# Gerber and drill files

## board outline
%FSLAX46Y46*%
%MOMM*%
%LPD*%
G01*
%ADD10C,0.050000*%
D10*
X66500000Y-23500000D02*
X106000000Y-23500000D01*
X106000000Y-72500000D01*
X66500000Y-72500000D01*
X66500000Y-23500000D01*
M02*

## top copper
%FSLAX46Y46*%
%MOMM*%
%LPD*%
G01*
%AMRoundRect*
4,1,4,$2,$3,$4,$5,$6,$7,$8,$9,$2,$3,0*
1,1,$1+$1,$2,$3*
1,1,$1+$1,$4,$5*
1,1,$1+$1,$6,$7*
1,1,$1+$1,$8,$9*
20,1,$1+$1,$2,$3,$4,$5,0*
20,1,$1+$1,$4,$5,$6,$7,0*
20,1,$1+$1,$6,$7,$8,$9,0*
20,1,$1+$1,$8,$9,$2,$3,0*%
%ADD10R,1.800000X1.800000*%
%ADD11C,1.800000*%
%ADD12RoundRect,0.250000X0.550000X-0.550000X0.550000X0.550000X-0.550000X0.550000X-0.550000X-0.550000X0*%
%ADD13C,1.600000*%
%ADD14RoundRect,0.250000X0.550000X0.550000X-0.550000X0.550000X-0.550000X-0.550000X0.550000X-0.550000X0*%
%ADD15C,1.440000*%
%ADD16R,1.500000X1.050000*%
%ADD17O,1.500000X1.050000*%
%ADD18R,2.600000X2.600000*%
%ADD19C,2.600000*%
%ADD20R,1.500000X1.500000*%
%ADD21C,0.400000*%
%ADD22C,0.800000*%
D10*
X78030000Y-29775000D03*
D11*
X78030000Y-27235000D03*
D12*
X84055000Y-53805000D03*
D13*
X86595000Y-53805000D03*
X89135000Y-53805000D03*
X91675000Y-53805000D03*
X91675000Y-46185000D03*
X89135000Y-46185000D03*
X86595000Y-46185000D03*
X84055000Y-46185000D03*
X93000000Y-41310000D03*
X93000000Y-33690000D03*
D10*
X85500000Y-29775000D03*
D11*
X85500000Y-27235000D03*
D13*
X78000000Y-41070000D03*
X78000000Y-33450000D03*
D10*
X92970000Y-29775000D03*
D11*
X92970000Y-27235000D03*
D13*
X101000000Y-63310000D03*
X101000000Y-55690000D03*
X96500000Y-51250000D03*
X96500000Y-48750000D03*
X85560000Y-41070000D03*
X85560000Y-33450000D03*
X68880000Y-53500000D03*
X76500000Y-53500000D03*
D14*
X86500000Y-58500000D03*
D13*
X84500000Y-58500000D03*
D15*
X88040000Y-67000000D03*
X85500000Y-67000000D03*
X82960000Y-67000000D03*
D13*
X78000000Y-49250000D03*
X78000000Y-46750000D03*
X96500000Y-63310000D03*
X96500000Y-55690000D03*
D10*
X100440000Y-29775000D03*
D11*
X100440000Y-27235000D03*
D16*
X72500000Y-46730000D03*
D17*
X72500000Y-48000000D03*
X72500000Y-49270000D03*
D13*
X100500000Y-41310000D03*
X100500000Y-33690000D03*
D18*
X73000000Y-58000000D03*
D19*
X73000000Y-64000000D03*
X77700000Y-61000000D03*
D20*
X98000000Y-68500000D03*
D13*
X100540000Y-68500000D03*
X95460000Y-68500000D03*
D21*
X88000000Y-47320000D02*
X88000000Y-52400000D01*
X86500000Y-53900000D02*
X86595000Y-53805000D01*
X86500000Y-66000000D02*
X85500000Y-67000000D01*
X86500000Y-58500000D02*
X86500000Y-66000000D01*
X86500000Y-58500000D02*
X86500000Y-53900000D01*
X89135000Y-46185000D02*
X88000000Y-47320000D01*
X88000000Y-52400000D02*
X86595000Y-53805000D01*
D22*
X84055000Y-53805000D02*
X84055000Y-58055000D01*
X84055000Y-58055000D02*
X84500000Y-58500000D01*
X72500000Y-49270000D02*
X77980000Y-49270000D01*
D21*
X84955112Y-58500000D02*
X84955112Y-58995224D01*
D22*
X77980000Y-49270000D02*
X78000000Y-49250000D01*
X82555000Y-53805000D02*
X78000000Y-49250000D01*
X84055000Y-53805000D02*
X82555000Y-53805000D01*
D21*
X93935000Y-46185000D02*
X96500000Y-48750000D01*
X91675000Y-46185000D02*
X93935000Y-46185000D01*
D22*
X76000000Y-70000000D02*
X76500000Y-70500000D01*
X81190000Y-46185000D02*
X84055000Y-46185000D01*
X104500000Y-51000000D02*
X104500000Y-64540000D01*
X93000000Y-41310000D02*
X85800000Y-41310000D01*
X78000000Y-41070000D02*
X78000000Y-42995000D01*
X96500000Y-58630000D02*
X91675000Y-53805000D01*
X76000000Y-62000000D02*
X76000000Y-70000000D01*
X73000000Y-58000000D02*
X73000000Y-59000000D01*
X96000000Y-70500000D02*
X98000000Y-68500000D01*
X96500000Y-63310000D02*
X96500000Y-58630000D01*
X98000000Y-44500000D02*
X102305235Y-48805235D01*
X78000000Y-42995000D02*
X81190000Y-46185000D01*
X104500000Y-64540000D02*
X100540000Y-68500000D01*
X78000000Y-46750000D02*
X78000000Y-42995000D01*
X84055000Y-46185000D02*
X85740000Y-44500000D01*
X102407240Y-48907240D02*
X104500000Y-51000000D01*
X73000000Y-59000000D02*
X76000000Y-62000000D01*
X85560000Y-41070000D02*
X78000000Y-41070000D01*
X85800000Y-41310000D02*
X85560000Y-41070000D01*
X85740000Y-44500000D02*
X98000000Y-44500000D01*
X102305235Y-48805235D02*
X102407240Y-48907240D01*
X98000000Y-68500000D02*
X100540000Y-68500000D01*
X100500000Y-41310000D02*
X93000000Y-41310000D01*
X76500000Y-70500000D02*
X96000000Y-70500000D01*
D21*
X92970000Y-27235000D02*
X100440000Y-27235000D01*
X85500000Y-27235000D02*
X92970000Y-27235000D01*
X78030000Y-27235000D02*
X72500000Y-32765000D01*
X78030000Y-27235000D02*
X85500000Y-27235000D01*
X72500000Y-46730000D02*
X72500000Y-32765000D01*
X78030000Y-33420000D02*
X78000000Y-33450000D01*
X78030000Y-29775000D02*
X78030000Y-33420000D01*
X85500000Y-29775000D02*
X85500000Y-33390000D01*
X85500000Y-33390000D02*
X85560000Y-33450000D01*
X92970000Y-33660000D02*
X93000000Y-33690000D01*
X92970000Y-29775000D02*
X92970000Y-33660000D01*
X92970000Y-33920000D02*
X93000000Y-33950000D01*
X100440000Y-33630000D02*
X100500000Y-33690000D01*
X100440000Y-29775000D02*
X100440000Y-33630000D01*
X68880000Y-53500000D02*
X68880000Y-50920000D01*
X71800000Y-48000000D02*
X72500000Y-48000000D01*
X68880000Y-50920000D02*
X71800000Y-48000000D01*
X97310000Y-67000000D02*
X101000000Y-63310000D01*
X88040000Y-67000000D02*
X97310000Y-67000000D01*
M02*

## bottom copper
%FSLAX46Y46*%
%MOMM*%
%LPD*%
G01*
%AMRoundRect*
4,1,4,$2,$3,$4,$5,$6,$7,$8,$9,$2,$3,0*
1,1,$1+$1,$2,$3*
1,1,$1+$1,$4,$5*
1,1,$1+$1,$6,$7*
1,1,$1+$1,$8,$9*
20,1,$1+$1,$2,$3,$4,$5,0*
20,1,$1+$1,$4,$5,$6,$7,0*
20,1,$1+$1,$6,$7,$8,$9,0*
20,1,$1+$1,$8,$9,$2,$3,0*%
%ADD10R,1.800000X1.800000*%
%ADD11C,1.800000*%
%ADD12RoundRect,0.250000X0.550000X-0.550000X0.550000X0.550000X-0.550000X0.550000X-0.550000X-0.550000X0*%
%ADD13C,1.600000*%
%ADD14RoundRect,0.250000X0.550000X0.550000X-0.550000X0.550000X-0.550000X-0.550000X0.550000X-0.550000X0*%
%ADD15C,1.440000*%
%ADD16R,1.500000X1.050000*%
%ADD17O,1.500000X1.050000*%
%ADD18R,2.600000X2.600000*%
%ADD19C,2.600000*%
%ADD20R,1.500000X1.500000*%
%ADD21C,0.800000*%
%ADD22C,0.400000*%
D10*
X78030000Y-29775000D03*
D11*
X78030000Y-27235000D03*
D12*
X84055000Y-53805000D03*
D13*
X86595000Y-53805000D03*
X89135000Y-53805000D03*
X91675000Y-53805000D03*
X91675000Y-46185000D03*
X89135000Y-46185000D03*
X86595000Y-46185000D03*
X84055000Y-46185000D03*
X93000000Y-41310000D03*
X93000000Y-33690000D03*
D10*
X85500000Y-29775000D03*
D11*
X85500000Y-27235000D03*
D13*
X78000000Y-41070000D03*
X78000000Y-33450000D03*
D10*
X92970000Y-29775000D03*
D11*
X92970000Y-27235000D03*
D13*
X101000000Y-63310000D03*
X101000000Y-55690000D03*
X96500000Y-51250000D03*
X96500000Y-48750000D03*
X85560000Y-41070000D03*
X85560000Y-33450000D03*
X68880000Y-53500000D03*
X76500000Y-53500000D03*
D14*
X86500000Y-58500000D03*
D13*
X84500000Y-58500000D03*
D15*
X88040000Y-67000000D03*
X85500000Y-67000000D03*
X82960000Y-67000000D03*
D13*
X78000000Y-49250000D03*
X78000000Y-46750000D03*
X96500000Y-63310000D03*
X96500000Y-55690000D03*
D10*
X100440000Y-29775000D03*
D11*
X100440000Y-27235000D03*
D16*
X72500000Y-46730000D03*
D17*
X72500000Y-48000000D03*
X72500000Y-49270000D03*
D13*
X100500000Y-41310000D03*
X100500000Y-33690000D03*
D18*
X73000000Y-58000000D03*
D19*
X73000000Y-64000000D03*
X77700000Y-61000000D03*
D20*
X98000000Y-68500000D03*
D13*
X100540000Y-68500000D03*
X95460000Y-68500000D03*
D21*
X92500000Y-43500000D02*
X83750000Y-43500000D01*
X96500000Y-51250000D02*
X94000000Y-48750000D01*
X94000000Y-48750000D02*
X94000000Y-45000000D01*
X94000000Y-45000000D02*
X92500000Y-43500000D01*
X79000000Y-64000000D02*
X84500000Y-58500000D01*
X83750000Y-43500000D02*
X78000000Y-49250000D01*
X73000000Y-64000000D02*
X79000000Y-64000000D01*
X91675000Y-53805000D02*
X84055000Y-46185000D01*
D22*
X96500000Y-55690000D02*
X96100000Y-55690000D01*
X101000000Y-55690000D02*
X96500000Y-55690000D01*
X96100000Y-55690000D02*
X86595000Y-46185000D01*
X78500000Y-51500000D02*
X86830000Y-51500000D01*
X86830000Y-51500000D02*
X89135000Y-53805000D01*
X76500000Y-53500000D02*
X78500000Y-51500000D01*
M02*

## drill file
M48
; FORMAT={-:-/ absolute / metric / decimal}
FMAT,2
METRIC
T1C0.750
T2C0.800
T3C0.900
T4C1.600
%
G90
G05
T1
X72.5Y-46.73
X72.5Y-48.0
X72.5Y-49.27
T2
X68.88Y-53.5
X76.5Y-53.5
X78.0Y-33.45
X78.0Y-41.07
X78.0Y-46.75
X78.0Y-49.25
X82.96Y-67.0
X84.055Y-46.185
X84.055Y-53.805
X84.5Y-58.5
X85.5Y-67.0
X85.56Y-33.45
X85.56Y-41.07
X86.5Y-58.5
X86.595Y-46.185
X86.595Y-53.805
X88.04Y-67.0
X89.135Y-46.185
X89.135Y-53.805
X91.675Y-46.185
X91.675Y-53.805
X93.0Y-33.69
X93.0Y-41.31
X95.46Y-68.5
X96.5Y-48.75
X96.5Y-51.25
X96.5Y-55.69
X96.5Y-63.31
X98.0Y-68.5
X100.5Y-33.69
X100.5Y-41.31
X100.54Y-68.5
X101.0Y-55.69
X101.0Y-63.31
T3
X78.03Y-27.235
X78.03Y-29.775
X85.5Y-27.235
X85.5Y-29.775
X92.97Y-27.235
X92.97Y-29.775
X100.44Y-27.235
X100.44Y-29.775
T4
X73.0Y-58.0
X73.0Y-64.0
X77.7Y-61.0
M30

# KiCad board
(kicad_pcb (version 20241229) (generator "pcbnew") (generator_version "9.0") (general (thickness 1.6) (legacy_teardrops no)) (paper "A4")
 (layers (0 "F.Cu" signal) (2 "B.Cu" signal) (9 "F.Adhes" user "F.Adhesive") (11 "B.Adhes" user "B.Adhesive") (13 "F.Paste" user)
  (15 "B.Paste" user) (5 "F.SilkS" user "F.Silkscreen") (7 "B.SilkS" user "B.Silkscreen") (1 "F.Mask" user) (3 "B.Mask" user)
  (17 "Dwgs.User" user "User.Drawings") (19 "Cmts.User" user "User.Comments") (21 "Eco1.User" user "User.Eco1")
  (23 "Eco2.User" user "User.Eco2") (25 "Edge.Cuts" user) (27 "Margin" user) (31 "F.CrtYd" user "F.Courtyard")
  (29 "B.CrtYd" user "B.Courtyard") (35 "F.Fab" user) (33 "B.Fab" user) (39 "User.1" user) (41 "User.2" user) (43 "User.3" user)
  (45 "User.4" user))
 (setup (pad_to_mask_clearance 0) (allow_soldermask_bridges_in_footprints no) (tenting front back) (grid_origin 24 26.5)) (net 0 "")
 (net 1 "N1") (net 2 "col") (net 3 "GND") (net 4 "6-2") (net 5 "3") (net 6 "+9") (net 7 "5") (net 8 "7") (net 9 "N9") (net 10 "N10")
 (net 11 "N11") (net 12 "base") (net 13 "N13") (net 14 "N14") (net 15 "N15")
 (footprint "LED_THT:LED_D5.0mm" (layer "F.Cu") (at 78.03 29.775 90)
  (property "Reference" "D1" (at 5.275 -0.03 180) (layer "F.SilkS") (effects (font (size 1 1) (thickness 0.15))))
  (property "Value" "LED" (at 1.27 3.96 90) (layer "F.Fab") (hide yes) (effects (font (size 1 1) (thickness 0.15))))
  (pad "1" thru_hole rect (at 0 0 90) (size 1.8 1.8) (drill 0.9) (layers "*.Cu" "*.Mask") (remove_unused_layers no) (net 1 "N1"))
  (pad "2" thru_hole circle (at 2.54 0 90) (size 1.8 1.8) (drill 0.9) (layers "*.Cu" "*.Mask") (remove_unused_layers no) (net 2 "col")))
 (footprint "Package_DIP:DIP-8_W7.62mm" (layer "F.Cu") (at 84.055 53.805 90)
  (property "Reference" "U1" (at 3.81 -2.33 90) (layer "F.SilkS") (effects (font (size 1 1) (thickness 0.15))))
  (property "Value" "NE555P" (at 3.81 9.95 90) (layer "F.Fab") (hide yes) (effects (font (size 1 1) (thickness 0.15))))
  (pad "1" thru_hole roundrect (at 0 0 90) (size 1.6 1.6) (drill 0.8) (layers "*.Cu" "*.Mask") (remove_unused_layers no)
   (roundrect_rratio 0.15625) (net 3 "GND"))
  (pad "2" thru_hole circle (at 0 2.54 90) (size 1.6 1.6) (drill 0.8) (layers "*.Cu" "*.Mask") (remove_unused_layers no) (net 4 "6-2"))
  (pad "3" thru_hole circle (at 0 5.08 90) (size 1.6 1.6) (drill 0.8) (layers "*.Cu" "*.Mask") (remove_unused_layers no) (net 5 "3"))
  (pad "4" thru_hole circle (at 0 7.62 90) (size 1.6 1.6) (drill 0.8) (layers "*.Cu" "*.Mask") (remove_unused_layers no) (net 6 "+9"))
  (pad "5" thru_hole circle (at 7.62 7.62 90) (size 1.6 1.6) (drill 0.8) (layers "*.Cu" "*.Mask") (remove_unused_layers no) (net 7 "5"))
  (pad "6" thru_hole circle (at 7.62 5.08 90) (size 1.6 1.6) (drill 0.8) (layers "*.Cu" "*.Mask") (remove_unused_layers no) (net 4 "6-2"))
  (pad "7" thru_hole circle (at 7.62 2.54 90) (size 1.6 1.6) (drill 0.8) (layers "*.Cu" "*.Mask") (remove_unused_layers no) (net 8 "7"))
  (pad "8" thru_hole circle (at 7.62 0 90) (size 1.6 1.6) (drill 0.8) (layers "*.Cu" "*.Mask") (remove_unused_layers no) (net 6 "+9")))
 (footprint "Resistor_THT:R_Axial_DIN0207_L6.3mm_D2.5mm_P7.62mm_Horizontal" (layer "F.Cu") (at 93 41.31 90)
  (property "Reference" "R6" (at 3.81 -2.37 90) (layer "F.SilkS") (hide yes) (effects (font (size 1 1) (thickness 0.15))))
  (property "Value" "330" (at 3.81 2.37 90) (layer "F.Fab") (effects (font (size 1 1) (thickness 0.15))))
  (pad "1" thru_hole circle (at 0 0 90) (size 1.6 1.6) (drill 0.8) (layers "*.Cu" "*.Mask") (remove_unused_layers no) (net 6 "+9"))
  (pad "2" thru_hole circle (at 7.62 0 90) (size 1.6 1.6) (drill 0.8) (layers "*.Cu" "*.Mask") (remove_unused_layers no) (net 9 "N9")))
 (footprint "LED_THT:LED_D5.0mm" (layer "F.Cu") (at 85.5 29.775 90)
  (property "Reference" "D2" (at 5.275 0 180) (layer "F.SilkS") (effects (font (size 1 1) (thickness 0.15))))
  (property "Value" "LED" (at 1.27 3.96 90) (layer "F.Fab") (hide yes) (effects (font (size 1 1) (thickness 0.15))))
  (pad "1" thru_hole rect (at 0 0 90) (size 1.8 1.8) (drill 0.9) (layers "*.Cu" "*.Mask") (remove_unused_layers no) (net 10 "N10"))
  (pad "2" thru_hole circle (at 2.54 0 90) (size 1.8 1.8) (drill 0.9) (layers "*.Cu" "*.Mask") (remove_unused_layers no) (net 2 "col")))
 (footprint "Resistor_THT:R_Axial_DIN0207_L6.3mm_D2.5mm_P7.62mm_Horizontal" (layer "F.Cu") (at 78 41.07 90)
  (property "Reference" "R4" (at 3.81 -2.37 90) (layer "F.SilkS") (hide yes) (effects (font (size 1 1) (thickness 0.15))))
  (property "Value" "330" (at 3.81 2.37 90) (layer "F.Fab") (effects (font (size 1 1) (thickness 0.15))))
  (pad "1" thru_hole circle (at 0 0 90) (size 1.6 1.6) (drill 0.8) (layers "*.Cu" "*.Mask") (remove_unused_layers no) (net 6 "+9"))
  (pad "2" thru_hole circle (at 7.62 0 90) (size 1.6 1.6) (drill 0.8) (layers "*.Cu" "*.Mask") (remove_unused_layers no) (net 1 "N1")))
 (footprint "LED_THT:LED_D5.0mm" (layer "F.Cu") (at 92.97 29.775 90)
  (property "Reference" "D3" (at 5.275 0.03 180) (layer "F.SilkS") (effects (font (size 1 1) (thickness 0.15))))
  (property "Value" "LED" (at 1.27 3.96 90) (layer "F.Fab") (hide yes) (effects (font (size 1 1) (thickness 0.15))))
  (pad "1" thru_hole rect (at 0 0 90) (size 1.8 1.8) (drill 0.9) (layers "*.Cu" "*.Mask") (remove_unused_layers no) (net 9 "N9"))
  (pad "2" thru_hole circle (at 2.54 0 90) (size 1.8 1.8) (drill 0.9) (layers "*.Cu" "*.Mask") (remove_unused_layers no) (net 2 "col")))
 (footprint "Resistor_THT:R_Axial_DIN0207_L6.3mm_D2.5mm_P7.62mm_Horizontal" (layer "F.Cu") (at 101 63.31 90)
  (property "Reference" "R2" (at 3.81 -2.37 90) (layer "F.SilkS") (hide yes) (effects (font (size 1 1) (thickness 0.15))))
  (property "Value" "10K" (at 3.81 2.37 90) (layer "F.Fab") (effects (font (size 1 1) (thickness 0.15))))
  (pad "1" thru_hole circle (at 0 0 90) (size 1.6 1.6) (drill 0.8) (layers "*.Cu" "*.Mask") (remove_unused_layers no) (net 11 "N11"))
  (pad "2" thru_hole circle (at 7.62 0 90) (size 1.6 1.6) (drill 0.8) (layers "*.Cu" "*.Mask") (remove_unused_layers no) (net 8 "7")))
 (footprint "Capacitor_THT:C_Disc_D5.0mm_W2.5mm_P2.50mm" (layer "F.Cu") (at 96.5 51.25 90)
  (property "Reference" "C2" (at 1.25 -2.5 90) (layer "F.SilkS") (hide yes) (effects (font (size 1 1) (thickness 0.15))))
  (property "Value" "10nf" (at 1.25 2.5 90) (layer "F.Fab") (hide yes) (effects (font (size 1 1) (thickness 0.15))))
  (pad "1" thru_hole circle (at 0 0 90) (size 1.6 1.6) (drill 0.8) (layers "*.Cu" "*.Mask") (remove_unused_layers no) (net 3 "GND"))
  (pad "2" thru_hole circle (at 2.5 0 90) (size 1.6 1.6) (drill 0.8) (layers "*.Cu" "*.Mask") (remove_unused_layers no) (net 7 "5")))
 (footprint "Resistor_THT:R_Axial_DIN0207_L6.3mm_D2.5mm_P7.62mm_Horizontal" (layer "F.Cu") (at 85.56 41.07 90)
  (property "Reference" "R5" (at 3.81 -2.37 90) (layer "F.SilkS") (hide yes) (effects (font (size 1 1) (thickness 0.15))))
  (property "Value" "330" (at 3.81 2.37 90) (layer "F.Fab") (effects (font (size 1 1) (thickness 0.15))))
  (pad "1" thru_hole circle (at 0 0 90) (size 1.6 1.6) (drill 0.8) (layers "*.Cu" "*.Mask") (remove_unused_layers no) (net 6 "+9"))
  (pad "2" thru_hole circle (at 7.62 0 90) (size 1.6 1.6) (drill 0.8) (layers "*.Cu" "*.Mask") (remove_unused_layers no) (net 10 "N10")))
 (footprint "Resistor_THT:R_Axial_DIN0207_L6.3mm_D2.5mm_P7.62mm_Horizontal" (layer "F.Cu") (at 68.88 53.5)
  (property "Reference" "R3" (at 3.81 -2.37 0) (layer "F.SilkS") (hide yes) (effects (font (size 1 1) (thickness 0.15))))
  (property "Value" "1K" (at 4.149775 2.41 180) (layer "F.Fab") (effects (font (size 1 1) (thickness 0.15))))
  (pad "1" thru_hole circle (at 0 0) (size 1.6 1.6) (drill 0.8) (layers "*.Cu" "*.Mask") (remove_unused_layers no) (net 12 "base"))
  (pad "2" thru_hole circle (at 7.62 0) (size 1.6 1.6) (drill 0.8) (layers "*.Cu" "*.Mask") (remove_unused_layers no) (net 5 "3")))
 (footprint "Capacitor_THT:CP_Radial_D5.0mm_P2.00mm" (layer "F.Cu") (at 86.5 58.5 180)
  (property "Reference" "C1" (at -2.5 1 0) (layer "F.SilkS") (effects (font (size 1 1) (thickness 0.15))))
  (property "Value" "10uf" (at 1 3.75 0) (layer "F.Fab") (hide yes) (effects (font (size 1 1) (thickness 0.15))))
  (pad "1" thru_hole roundrect (at 0 0 180) (size 1.6 1.6) (drill 0.8) (layers "*.Cu" "*.Mask") (remove_unused_layers no)
   (roundrect_rratio 0.15625) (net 4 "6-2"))
  (pad "2" thru_hole circle (at 2 0 180) (size 1.6 1.6) (drill 0.8) (layers "*.Cu" "*.Mask") (remove_unused_layers no) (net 3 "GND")))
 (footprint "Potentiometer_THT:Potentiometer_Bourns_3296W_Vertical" (layer "F.Cu") (at 88.04 67)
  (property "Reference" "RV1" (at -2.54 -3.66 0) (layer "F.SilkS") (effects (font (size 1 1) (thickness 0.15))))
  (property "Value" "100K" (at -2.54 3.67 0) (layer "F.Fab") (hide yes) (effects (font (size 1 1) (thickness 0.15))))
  (pad "1" thru_hole circle (at 0 0) (size 1.44 1.44) (drill 0.8) (layers "*.Cu" "*.Mask") (remove_unused_layers no) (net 11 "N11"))
  (pad "2" thru_hole circle (at -2.54 0) (size 1.44 1.44) (drill 0.8) (layers "*.Cu" "*.Mask") (remove_unused_layers no) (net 4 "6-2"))
  (pad "3" thru_hole circle (at -5.08 0) (size 1.44 1.44) (drill 0.8) (layers "*.Cu" "*.Mask") (remove_unused_layers no) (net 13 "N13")))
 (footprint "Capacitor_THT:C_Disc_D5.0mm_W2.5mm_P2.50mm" (layer "F.Cu") (at 78 49.25 90)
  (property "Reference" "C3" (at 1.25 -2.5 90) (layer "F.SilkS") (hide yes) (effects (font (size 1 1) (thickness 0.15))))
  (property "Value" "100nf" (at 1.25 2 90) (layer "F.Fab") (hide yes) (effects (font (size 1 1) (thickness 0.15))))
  (pad "1" thru_hole circle (at 0 0 90) (size 1.6 1.6) (drill 0.8) (layers "*.Cu" "*.Mask") (remove_unused_layers no) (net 3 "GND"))
  (pad "2" thru_hole circle (at 2.5 0 90) (size 1.6 1.6) (drill 0.8) (layers "*.Cu" "*.Mask") (remove_unused_layers no) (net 6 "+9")))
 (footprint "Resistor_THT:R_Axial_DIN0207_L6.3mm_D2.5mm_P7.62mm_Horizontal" (layer "F.Cu") (at 96.5 63.31 90)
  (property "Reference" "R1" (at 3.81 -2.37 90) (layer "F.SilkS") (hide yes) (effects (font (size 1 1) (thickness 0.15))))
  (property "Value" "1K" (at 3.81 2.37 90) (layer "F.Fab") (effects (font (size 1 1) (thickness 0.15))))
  (pad "1" thru_hole circle (at 0 0 90) (size 1.6 1.6) (drill 0.8) (layers "*.Cu" "*.Mask") (remove_unused_layers no) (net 6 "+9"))
  (pad "2" thru_hole circle (at 7.62 0 90) (size 1.6 1.6) (drill 0.8) (layers "*.Cu" "*.Mask") (remove_unused_layers no) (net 8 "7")))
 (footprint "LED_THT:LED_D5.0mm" (layer "F.Cu") (at 100.44 29.775 90)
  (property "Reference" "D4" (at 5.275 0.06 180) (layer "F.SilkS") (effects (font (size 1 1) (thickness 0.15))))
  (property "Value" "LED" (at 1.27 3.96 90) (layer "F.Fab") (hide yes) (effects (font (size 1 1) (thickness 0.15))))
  (pad "1" thru_hole rect (at 0 0 90) (size 1.8 1.8) (drill 0.9) (layers "*.Cu" "*.Mask") (remove_unused_layers no) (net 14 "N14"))
  (pad "2" thru_hole circle (at 2.54 0 90) (size 1.8 1.8) (drill 0.9) (layers "*.Cu" "*.Mask") (remove_unused_layers no) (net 2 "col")))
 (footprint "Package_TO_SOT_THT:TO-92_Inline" (layer "F.Cu") (at 72.5 46.73 -90)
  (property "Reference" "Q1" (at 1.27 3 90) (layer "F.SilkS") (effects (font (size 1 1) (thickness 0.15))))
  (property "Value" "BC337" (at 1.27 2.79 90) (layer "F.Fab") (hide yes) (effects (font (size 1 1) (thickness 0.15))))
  (pad "1" thru_hole rect (at 0 0 270) (size 1.05 1.5) (drill 0.75) (layers "*.Cu" "*.Mask") (remove_unused_layers no) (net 2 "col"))
  (pad "2" thru_hole oval (at 1.27 0 270) (size 1.05 1.5) (drill 0.75) (layers "*.Cu" "*.Mask") (remove_unused_layers no) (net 12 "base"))
  (pad "3" thru_hole oval (at 2.54 0 270) (size 1.05 1.5) (drill 0.75) (layers "*.Cu" "*.Mask") (remove_unused_layers no) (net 3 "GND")))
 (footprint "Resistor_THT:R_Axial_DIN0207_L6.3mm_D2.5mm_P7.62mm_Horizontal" (layer "F.Cu") (at 100.5 41.31 90)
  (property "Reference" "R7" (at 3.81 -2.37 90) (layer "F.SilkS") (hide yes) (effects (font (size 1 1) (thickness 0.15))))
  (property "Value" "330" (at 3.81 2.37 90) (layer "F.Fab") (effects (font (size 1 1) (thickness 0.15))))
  (pad "1" thru_hole circle (at 0 0 90) (size 1.6 1.6) (drill 0.8) (layers "*.Cu" "*.Mask") (remove_unused_layers no) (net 6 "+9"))
  (pad "2" thru_hole circle (at 7.62 0 90) (size 1.6 1.6) (drill 0.8) (layers "*.Cu" "*.Mask") (remove_unused_layers no) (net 14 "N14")))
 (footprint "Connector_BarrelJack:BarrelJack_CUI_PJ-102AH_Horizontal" (layer "F.Cu") (at 73 58)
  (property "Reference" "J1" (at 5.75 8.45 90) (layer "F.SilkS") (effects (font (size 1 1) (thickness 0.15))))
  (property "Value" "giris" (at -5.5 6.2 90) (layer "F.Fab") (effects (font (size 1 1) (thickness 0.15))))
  (pad "1" thru_hole rect (at 0 0) (size 2.6 2.6) (drill 1.6) (layers "*.Cu" "*.Mask") (remove_unused_layers no) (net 6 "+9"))
  (pad "2" thru_hole circle (at 0 6) (size 2.6 2.6) (drill 1.6) (layers "*.Cu" "*.Mask") (remove_unused_layers no) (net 3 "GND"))
  (pad "3" thru_hole circle (at 4.7 3) (size 2.6 2.6) (drill 1.6) (layers "*.Cu" "*.Mask") (remove_unused_layers no)))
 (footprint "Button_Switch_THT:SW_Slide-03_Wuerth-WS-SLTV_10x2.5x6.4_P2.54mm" (layer "F.Cu") (at 98 68.5 180)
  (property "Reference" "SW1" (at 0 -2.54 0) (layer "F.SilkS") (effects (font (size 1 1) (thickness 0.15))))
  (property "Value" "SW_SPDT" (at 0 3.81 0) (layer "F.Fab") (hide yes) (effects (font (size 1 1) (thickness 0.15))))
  (pad "1" thru_hole rect (at 0 0 180) (size 1.5 1.5) (drill 0.8) (layers "*.Cu" "*.Mask") (remove_unused_layers no) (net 6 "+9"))
  (pad "2" thru_hole circle (at -2.54 0 180) (size 1.6 1.6) (drill 0.8) (layers "*.Cu" "*.Mask") (remove_unused_layers no) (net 6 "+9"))
  (pad "3" thru_hole circle (at 2.54 0 180) (size 1.6 1.6) (drill 0.8) (layers "*.Cu" "*.Mask") (remove_unused_layers no) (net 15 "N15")))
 (gr_rect (start 66.5 23.5) (end 106 72.5) (stroke (width 0.05) (type default)) (fill no) (layer "Edge.Cuts"))
 (segment (start 88 47.32) (end 88 52.4) (width 0.4) (layer "F.Cu") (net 4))
 (segment (start 86.5 53.9) (end 86.595 53.805) (width 0.4) (layer "F.Cu") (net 4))
 (segment (start 86.5 66) (end 85.5 67) (width 0.4) (layer "F.Cu") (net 4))
 (segment (start 86.5 58.5) (end 86.5 66) (width 0.4) (layer "F.Cu") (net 4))
 (segment (start 86.5 58.5) (end 86.5 53.9) (width 0.4) (layer "F.Cu") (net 4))
 (segment (start 89.135 46.185) (end 88 47.32) (width 0.4) (layer "F.Cu") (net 4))
 (segment (start 88 52.4) (end 86.595 53.805) (width 0.4) (layer "F.Cu") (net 4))
 (segment (start 84.055 53.805) (end 84.055 58.055) (width 0.8) (layer "F.Cu") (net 3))
 (segment (start 84.055 58.055) (end 84.5 58.5) (width 0.8) (layer "F.Cu") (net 3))
 (segment (start 72.5 49.27) (end 77.98 49.27) (width 0.8) (layer "F.Cu") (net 3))
 (segment (start 84.955112 58.5) (end 84.955112 58.995224) (width 0.4) (layer "F.Cu") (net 3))
 (segment (start 77.98 49.27) (end 78 49.25) (width 0.8) (layer "F.Cu") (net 3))
 (segment (start 82.555 53.805) (end 78 49.25) (width 0.8) (layer "F.Cu") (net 3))
 (segment (start 84.055 53.805) (end 82.555 53.805) (width 0.8) (layer "F.Cu") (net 3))
 (segment (start 92.5 43.5) (end 83.75 43.5) (width 0.8) (layer "B.Cu") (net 3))
 (segment (start 96.5 51.25) (end 94 48.75) (width 0.8) (layer "B.Cu") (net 3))
 (segment (start 94 48.75) (end 94 45) (width 0.8) (layer "B.Cu") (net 3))
 (segment (start 94 45) (end 92.5 43.5) (width 0.8) (layer "B.Cu") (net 3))
 (segment (start 79 64) (end 84.5 58.5) (width 0.8) (layer "B.Cu") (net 3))
 (segment (start 83.75 43.5) (end 78 49.25) (width 0.8) (layer "B.Cu") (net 3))
 (segment (start 73 64) (end 79 64) (width 0.8) (layer "B.Cu") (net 3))
 (segment (start 93.935 46.185) (end 96.5 48.75) (width 0.4) (layer "F.Cu") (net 7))
 (segment (start 91.675 46.185) (end 93.935 46.185) (width 0.4) (layer "F.Cu") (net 7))
 (segment (start 76 70) (end 76.5 70.5) (width 0.8) (layer "F.Cu") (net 6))
 (segment (start 81.19 46.185) (end 84.055 46.185) (width 0.8) (layer "F.Cu") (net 6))
 (segment (start 104.5 51) (end 104.5 64.54) (width 0.8) (layer "F.Cu") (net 6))
 (segment (start 93 41.31) (end 85.8 41.31) (width 0.8) (layer "F.Cu") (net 6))
 (segment (start 78 41.07) (end 78 42.995) (width 0.8) (layer "F.Cu") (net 6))
 (segment (start 96.5 58.63) (end 91.675 53.805) (width 0.8) (layer "F.Cu") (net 6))
 (segment (start 76 62) (end 76 70) (width 0.8) (layer "F.Cu") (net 6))
 (segment (start 73 58) (end 73 59) (width 0.8) (layer "F.Cu") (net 6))
 (segment (start 96 70.5) (end 98 68.5) (width 0.8) (layer "F.Cu") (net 6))
 (segment (start 96.5 63.31) (end 96.5 58.63) (width 0.8) (layer "F.Cu") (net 6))
 (segment (start 98 44.5) (end 102.305235 48.805235) (width 0.8) (layer "F.Cu") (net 6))
 (segment (start 78 42.995) (end 81.19 46.185) (width 0.8) (layer "F.Cu") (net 6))
 (segment (start 104.5 64.54) (end 100.54 68.5) (width 0.8) (layer "F.Cu") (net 6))
 (segment (start 78 46.75) (end 78 42.995) (width 0.8) (layer "F.Cu") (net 6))
 (segment (start 84.055 46.185) (end 85.74 44.5) (width 0.8) (layer "F.Cu") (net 6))
 (segment (start 102.40724 48.90724) (end 104.5 51) (width 0.8) (layer "F.Cu") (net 6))
 (segment (start 73 59) (end 76 62) (width 0.8) (layer "F.Cu") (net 6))
 (segment (start 85.56 41.07) (end 78 41.07) (width 0.8) (layer "F.Cu") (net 6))
 (segment (start 85.8 41.31) (end 85.56 41.07) (width 0.8) (layer "F.Cu") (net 6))
 (segment (start 85.74 44.5) (end 98 44.5) (width 0.8) (layer "F.Cu") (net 6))
 (segment (start 102.305235 48.805235) (end 102.40724 48.90724) (width 0.8) (layer "F.Cu") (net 6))
 (segment (start 98 68.5) (end 100.54 68.5) (width 0.8) (layer "F.Cu") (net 6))
 (segment (start 100.5 41.31) (end 93 41.31) (width 0.8) (layer "F.Cu") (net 6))
 (segment (start 76.5 70.5) (end 96 70.5) (width 0.8) (layer "F.Cu") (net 6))
 (segment (start 91.675 53.805) (end 84.055 46.185) (width 0.8) (layer "B.Cu") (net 6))
 (segment (start 92.97 27.235) (end 100.44 27.235) (width 0.4) (layer "F.Cu") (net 2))
 (segment (start 85.5 27.235) (end 92.97 27.235) (width 0.4) (layer "F.Cu") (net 2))
 (segment (start 78.03 27.235) (end 72.5 32.765) (width 0.4) (layer "F.Cu") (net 2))
 (segment (start 78.03 27.235) (end 85.5 27.235) (width 0.4) (layer "F.Cu") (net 2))
 (segment (start 72.5 46.73) (end 72.5 32.765) (width 0.4) (layer "F.Cu") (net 2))
 (segment (start 78.03 33.42) (end 78 33.45) (width 0.4) (layer "F.Cu") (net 1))
 (segment (start 78.03 29.775) (end 78.03 33.42) (width 0.4) (layer "F.Cu") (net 1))
 (segment (start 85.5 29.775) (end 85.5 33.39) (width 0.4) (layer "F.Cu") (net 10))
 (segment (start 85.5 33.39) (end 85.56 33.45) (width 0.4) (layer "F.Cu") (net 10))
 (segment (start 92.97 33.66) (end 93 33.69) (width 0.4) (layer "F.Cu") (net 9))
 (segment (start 92.97 29.775) (end 92.97 33.66) (width 0.4) (layer "F.Cu") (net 9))
 (segment (start 92.97 33.92) (end 93 33.95) (width 0.4) (layer "F.Cu") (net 9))
 (segment (start 100.44 33.63) (end 100.5 33.69) (width 0.4) (layer "F.Cu") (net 14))
 (segment (start 100.44 29.775) (end 100.44 33.63) (width 0.4) (layer "F.Cu") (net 14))
 (segment (start 68.88 53.5) (end 68.88 50.92) (width 0.4) (layer "F.Cu") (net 12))
 (segment (start 71.8 48) (end 72.5 48) (width 0.4) (layer "F.Cu") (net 12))
 (segment (start 68.88 50.92) (end 71.8 48) (width 0.4) (layer "F.Cu") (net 12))
 (segment (start 96.5 55.69) (end 96.1 55.69) (width 0.4) (layer "B.Cu") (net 8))
 (segment (start 101 55.69) (end 96.5 55.69) (width 0.4) (layer "B.Cu") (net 8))
 (segment (start 96.1 55.69) (end 86.595 46.185) (width 0.4) (layer "B.Cu") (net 8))
 (segment (start 97.31 67) (end 101 63.31) (width 0.4) (layer "F.Cu") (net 11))
 (segment (start 88.04 67) (end 97.31 67) (width 0.4) (layer "F.Cu") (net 11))
 (segment (start 78.5 51.5) (end 86.83 51.5) (width 0.4) (layer "B.Cu") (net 5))
 (segment (start 86.83 51.5) (end 89.135 53.805) (width 0.4) (layer "B.Cu") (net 5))
 (segment (start 76.5 53.5) (end 78.5 51.5) (width 0.4) (layer "B.Cu") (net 5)))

